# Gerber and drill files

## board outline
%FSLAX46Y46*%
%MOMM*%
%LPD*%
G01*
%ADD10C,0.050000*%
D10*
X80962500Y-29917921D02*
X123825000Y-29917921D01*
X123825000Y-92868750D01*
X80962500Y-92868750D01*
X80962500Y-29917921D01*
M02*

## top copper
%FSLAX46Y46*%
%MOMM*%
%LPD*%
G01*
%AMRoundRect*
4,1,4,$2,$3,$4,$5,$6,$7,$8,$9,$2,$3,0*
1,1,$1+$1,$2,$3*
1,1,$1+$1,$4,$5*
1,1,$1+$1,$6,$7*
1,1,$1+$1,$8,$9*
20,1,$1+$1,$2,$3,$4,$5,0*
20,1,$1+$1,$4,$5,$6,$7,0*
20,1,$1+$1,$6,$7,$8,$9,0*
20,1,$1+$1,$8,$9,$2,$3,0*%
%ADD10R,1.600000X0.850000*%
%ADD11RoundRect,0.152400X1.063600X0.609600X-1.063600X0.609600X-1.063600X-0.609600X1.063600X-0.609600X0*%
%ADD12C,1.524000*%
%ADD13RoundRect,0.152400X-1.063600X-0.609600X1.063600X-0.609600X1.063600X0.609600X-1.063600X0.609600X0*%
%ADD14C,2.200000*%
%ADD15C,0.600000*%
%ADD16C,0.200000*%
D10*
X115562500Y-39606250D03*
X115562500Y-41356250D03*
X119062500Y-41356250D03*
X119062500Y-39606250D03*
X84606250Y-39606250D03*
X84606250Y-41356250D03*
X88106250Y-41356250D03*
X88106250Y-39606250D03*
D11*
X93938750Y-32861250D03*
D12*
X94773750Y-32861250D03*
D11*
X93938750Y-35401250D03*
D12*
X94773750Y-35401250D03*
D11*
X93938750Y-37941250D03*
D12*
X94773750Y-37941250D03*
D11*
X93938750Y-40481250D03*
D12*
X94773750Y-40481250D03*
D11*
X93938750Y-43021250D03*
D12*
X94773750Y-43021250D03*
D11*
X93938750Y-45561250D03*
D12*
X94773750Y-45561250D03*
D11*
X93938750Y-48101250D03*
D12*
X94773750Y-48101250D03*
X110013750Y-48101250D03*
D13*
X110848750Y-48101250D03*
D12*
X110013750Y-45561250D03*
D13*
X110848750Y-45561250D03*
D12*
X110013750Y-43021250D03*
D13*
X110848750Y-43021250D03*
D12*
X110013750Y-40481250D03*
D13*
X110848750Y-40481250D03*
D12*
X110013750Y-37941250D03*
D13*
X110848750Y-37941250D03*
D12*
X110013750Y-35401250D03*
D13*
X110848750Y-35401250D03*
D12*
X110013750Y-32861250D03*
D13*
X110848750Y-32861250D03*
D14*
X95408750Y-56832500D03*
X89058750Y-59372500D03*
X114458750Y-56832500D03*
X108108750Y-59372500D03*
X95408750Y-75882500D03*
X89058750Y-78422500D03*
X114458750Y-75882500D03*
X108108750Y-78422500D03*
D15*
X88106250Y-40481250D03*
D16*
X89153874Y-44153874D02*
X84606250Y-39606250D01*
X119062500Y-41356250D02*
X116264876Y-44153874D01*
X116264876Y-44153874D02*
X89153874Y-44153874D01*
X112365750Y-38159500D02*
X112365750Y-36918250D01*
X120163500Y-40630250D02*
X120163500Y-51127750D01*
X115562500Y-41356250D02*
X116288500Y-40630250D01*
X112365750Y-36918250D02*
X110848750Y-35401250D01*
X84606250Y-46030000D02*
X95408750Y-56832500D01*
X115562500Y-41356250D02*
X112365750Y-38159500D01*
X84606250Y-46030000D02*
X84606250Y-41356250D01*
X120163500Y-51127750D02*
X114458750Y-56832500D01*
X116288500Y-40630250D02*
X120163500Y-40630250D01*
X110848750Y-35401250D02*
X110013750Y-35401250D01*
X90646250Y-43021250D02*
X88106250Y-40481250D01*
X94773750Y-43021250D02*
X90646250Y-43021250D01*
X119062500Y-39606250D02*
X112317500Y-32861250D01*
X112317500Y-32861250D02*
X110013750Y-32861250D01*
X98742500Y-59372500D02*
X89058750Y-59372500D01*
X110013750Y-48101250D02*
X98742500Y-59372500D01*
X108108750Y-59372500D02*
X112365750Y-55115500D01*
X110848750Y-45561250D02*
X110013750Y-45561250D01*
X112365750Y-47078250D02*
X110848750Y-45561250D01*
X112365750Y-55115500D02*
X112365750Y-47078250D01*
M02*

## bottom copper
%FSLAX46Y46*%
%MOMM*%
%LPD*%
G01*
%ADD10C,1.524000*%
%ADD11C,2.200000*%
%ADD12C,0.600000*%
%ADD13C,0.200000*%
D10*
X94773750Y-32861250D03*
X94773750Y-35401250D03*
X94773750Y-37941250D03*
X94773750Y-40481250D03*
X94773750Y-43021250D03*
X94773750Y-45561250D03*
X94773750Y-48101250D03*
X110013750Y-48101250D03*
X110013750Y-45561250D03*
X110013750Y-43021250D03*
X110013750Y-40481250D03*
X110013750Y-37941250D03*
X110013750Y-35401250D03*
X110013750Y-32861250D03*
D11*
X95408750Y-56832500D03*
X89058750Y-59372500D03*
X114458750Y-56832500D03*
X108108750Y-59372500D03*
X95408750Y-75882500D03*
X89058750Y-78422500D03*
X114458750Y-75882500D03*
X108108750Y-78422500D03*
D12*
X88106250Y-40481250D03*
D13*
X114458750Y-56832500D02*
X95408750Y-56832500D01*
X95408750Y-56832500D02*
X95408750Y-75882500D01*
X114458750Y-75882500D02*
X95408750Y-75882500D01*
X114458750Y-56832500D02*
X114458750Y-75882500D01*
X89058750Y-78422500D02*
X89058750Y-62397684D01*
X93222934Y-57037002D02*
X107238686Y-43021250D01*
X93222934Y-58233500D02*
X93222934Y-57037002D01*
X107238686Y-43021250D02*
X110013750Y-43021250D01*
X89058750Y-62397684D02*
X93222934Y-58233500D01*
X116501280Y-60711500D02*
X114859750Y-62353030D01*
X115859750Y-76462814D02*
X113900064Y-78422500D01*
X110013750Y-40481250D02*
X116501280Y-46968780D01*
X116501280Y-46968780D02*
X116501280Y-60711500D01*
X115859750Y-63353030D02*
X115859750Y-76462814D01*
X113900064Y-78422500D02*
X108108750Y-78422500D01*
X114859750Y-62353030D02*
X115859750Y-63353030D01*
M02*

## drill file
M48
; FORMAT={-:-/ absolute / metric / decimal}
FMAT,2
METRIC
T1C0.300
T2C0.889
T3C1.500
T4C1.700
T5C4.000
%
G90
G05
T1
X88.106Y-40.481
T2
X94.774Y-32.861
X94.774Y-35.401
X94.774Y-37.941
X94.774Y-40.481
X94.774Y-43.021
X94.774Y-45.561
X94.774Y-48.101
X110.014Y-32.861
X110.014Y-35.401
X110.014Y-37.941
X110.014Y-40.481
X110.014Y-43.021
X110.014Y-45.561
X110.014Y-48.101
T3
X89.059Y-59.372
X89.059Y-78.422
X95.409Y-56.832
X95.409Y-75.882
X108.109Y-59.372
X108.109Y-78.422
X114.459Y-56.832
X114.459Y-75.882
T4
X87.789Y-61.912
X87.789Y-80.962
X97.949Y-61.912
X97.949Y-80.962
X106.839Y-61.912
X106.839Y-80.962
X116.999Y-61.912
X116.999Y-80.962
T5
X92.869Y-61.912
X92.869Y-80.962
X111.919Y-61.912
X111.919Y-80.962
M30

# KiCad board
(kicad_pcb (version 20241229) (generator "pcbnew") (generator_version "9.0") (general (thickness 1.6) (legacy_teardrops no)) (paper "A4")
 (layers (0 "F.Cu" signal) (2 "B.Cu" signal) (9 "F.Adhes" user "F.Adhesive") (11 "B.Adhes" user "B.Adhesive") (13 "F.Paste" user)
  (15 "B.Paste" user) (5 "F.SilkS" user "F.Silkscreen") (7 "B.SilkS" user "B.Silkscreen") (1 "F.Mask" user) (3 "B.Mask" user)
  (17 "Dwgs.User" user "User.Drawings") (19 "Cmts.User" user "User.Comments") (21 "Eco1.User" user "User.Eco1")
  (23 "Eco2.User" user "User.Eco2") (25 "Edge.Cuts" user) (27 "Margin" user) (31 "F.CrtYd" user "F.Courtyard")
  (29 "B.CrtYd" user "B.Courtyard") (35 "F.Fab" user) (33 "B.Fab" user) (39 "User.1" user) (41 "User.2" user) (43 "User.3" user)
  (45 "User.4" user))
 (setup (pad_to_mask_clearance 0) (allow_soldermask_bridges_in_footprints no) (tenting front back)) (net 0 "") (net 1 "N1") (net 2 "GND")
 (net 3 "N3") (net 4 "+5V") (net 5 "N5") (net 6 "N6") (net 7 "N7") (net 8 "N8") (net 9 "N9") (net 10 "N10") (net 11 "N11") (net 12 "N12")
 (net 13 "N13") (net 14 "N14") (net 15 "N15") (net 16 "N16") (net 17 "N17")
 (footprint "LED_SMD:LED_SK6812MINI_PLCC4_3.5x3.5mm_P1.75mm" (layer "F.Cu") (at 117.3125 40.48125)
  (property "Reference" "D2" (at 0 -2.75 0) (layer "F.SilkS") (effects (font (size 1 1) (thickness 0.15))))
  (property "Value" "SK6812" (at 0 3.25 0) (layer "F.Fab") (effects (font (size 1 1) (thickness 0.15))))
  (pad "1" smd rect (at -1.75 -0.875) (size 1.6 0.85) (layers "F.Cu" "F.Mask" "F.Paste") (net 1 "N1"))
  (pad "2" smd rect (at -1.75 0.875) (size 1.6 0.85) (layers "F.Cu" "F.Mask" "F.Paste") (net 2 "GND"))
  (pad "3" smd rect (at 1.75 0.875) (size 1.6 0.85) (layers "F.Cu" "F.Mask" "F.Paste") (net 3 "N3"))
  (pad "4" smd rect (at 1.75 -0.875) (size 1.6 0.85) (layers "F.Cu" "F.Mask" "F.Paste") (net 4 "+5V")))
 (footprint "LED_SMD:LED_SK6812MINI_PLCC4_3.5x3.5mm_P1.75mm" (layer "F.Cu") (at 86.35625 40.48125)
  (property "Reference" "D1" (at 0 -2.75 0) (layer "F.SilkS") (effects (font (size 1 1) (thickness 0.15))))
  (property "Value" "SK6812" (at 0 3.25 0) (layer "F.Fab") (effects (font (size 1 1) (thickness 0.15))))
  (pad "1" smd rect (at -1.75 -0.875) (size 1.6 0.85) (layers "F.Cu" "F.Mask" "F.Paste") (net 3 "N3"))
  (pad "2" smd rect (at -1.75 0.875) (size 1.6 0.85) (layers "F.Cu" "F.Mask" "F.Paste") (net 2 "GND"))
  (pad "3" smd rect (at 1.75 0.875) (size 1.6 0.85) (layers "F.Cu" "F.Mask" "F.Paste") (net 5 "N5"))
  (pad "4" smd rect (at 1.75 -0.875) (size 1.6 0.85) (layers "F.Cu" "F.Mask" "F.Paste") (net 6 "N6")))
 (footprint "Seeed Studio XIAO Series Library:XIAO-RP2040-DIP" (layer "F.Cu") (at 102.39375 40.48125)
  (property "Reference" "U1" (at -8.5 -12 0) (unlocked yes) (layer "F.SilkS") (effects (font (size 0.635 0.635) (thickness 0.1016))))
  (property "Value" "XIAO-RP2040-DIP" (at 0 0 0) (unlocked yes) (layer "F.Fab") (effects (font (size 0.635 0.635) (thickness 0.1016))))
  (pad "1" smd roundrect (at -8.455 -7.62 180) (size 2.432 1.524) (layers "F.Cu" "F.Mask") (roundrect_rratio 0.1) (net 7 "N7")
   (thermal_bridge_angle 45))
  (pad "1" thru_hole circle (at -7.62 -7.62 180) (size 1.524 1.524) (drill 0.889) (layers "*.Cu" "*.Mask") (remove_unused_layers no)
   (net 7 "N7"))
  (pad "2" smd roundrect (at -8.455 -5.08 180) (size 2.432 1.524) (layers "F.Cu" "F.Mask") (roundrect_rratio 0.1) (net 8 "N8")
   (thermal_bridge_angle 45))
  (pad "2" thru_hole circle (at -7.62 -5.08 180) (size 1.524 1.524) (drill 0.889) (layers "*.Cu" "*.Mask") (remove_unused_layers no)
   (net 8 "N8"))
  (pad "3" smd roundrect (at -8.455 -2.54 180) (size 2.432 1.524) (layers "F.Cu" "F.Mask") (roundrect_rratio 0.1) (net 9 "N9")
   (thermal_bridge_angle 45))
  (pad "3" thru_hole circle (at -7.62 -2.54 180) (size 1.524 1.524) (drill 0.889) (layers "*.Cu" "*.Mask") (remove_unused_layers no)
   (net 9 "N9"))
  (pad "4" smd roundrect (at -8.455 0 180) (size 2.432 1.524) (layers "F.Cu" "F.Mask") (roundrect_rratio 0.1) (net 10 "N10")
   (thermal_bridge_angle 45))
  (pad "4" thru_hole circle (at -7.62 0 180) (size 1.524 1.524) (drill 0.889) (layers "*.Cu" "*.Mask") (remove_unused_layers no)
   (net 10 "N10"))
  (pad "5" smd roundrect (at -8.455 2.54 180) (size 2.432 1.524) (layers "F.Cu" "F.Mask") (roundrect_rratio 0.1) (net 5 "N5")
   (thermal_bridge_angle 45))
  (pad "5" thru_hole circle (at -7.62 2.54 180) (size 1.524 1.524) (drill 0.889) (layers "*.Cu" "*.Mask") (remove_unused_layers no)
   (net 5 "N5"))
  (pad "6" smd roundrect (at -8.455 5.08 180) (size 2.432 1.524) (layers "F.Cu" "F.Mask") (roundrect_rratio 0.1) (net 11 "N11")
   (thermal_bridge_angle 45))
  (pad "6" thru_hole circle (at -7.62 5.08 180) (size 1.524 1.524) (drill 0.889) (layers "*.Cu" "*.Mask") (remove_unused_layers no)
   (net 11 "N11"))
  (pad "7" smd roundrect (at -8.455 7.62 180) (size 2.432 1.524) (layers "F.Cu" "F.Mask") (roundrect_rratio 0.1) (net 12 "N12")
   (thermal_bridge_angle 45))
  (pad "7" thru_hole circle (at -7.62 7.62 180) (size 1.524 1.524) (drill 0.889) (layers "*.Cu" "*.Mask") (remove_unused_layers no)
   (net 12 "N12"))
  (pad "8" thru_hole circle (at 7.62 7.62) (size 1.524 1.524) (drill 0.889) (layers "*.Cu" "*.Mask") (remove_unused_layers no)
   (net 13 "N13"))
  (pad "8" smd roundrect (at 8.455 7.62) (size 2.432 1.524) (layers "F.Cu" "F.Mask") (roundrect_rratio 0.1) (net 13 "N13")
   (thermal_bridge_angle 45))
  (pad "9" thru_hole circle (at 7.62 5.08) (size 1.524 1.524) (drill 0.889) (layers "*.Cu" "*.Mask") (remove_unused_layers no)
   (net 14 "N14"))
  (pad "9" smd roundrect (at 8.455 5.08) (size 2.432 1.524) (layers "F.Cu" "F.Mask") (roundrect_rratio 0.1) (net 14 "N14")
   (thermal_bridge_angle 45))
  (pad "10" thru_hole circle (at 7.62 2.54) (size 1.524 1.524) (drill 0.889) (layers "*.Cu" "*.Mask") (remove_unused_layers no)
   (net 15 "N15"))
  (pad "10" smd roundrect (at 8.455 2.54) (size 2.432 1.524) (layers "F.Cu" "F.Mask") (roundrect_rratio 0.1) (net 15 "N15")
   (thermal_bridge_angle 45))
  (pad "11" thru_hole circle (at 7.62 0) (size 1.524 1.524) (drill 0.889) (layers "*.Cu" "*.Mask") (remove_unused_layers no) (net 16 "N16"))
  (pad "11" smd roundrect (at 8.455 0) (size 2.432 1.524) (layers "F.Cu" "F.Mask") (roundrect_rratio 0.1) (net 16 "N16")
   (thermal_bridge_angle 45))
  (pad "12" thru_hole circle (at 7.62 -2.54) (size 1.524 1.524) (drill 0.889) (layers "*.Cu" "*.Mask") (remove_unused_layers no)
   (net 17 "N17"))
  (pad "12" smd roundrect (at 8.455 -2.54) (size 2.432 1.524) (layers "F.Cu" "F.Mask") (roundrect_rratio 0.1) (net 17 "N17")
   (thermal_bridge_angle 45))
  (pad "13" thru_hole circle (at 7.62 -5.08) (size 1.524 1.524) (drill 0.889) (layers "*.Cu" "*.Mask") (remove_unused_layers no)
   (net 2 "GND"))
  (pad "13" smd roundrect (at 8.455 -5.08) (size 2.432 1.524) (layers "F.Cu" "F.Mask") (roundrect_rratio 0.1) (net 2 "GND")
   (thermal_bridge_angle 45))
  (pad "14" thru_hole circle (at 7.62 -7.62) (size 1.524 1.524) (drill 0.889) (layers "*.Cu" "*.Mask") (remove_unused_layers no)
   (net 4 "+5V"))
  (pad "14" smd roundrect (at 8.455 -7.62) (size 2.432 1.524) (layers "F.Cu" "F.Mask") (roundrect_rratio 0.1) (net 4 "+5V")
   (thermal_bridge_angle 45)))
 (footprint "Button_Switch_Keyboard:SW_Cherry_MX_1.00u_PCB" (layer "F.Cu") (at 95.40875 56.8325)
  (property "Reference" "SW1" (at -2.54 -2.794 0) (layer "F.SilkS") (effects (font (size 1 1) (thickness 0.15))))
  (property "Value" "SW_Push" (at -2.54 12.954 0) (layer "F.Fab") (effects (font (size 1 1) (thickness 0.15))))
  (pad "" np_thru_hole circle (at -7.62 5.08) (size 1.7 1.7) (drill 1.7) (layers "*.Cu" "*.Mask"))
  (pad "" np_thru_hole circle (at -2.54 5.08) (size 4 4) (drill 4) (layers "*.Cu" "*.Mask"))
  (pad "" np_thru_hole circle (at 2.54 5.08) (size 1.7 1.7) (drill 1.7) (layers "*.Cu" "*.Mask"))
  (pad "1" thru_hole circle (at 0 0) (size 2.2 2.2) (drill 1.5) (layers "*.Cu" "*.Mask") (remove_unused_layers no) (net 2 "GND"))
  (pad "2" thru_hole circle (at -6.35 2.54) (size 2.2 2.2) (drill 1.5) (layers "*.Cu" "*.Mask") (remove_unused_layers no) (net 13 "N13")))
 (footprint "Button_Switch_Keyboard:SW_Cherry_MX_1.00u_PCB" (layer "F.Cu") (at 114.45875 56.8325)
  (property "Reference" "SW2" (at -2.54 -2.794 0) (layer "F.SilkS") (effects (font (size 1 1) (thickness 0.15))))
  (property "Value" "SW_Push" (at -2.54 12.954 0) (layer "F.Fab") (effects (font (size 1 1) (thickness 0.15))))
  (pad "" np_thru_hole circle (at -7.62 5.08) (size 1.7 1.7) (drill 1.7) (layers "*.Cu" "*.Mask"))
  (pad "" np_thru_hole circle (at -2.54 5.08) (size 4 4) (drill 4) (layers "*.Cu" "*.Mask"))
  (pad "" np_thru_hole circle (at 2.54 5.08) (size 1.7 1.7) (drill 1.7) (layers "*.Cu" "*.Mask"))
  (pad "1" thru_hole circle (at 0 0) (size 2.2 2.2) (drill 1.5) (layers "*.Cu" "*.Mask") (remove_unused_layers no) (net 2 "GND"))
  (pad "2" thru_hole circle (at -6.35 2.54) (size 2.2 2.2) (drill 1.5) (layers "*.Cu" "*.Mask") (remove_unused_layers no) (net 14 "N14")))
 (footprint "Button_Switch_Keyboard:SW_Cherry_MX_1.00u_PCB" (layer "F.Cu") (at 95.40875 75.8825)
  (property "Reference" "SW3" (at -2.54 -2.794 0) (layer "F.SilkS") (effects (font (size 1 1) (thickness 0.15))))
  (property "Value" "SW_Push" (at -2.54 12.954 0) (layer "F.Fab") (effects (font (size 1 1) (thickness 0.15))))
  (pad "" np_thru_hole circle (at -7.62 5.08) (size 1.7 1.7) (drill 1.7) (layers "*.Cu" "*.Mask"))
  (pad "" np_thru_hole circle (at -2.54 5.08) (size 4 4) (drill 4) (layers "*.Cu" "*.Mask"))
  (pad "" np_thru_hole circle (at 2.54 5.08) (size 1.7 1.7) (drill 1.7) (layers "*.Cu" "*.Mask"))
  (pad "1" thru_hole circle (at 0 0) (size 2.2 2.2) (drill 1.5) (layers "*.Cu" "*.Mask") (remove_unused_layers no) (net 2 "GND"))
  (pad "2" thru_hole circle (at -6.35 2.54) (size 2.2 2.2) (drill 1.5) (layers "*.Cu" "*.Mask") (remove_unused_layers no) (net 15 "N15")))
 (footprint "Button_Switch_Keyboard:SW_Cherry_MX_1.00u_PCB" (layer "F.Cu") (at 114.45875 75.8825)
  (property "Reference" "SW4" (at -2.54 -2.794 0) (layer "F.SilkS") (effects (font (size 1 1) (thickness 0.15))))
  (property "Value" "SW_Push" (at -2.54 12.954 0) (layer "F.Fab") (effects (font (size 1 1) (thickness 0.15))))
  (pad "" np_thru_hole circle (at -7.62 5.08) (size 1.7 1.7) (drill 1.7) (layers "*.Cu" "*.Mask"))
  (pad "" np_thru_hole circle (at -2.54 5.08) (size 4 4) (drill 4) (layers "*.Cu" "*.Mask"))
  (pad "" np_thru_hole circle (at 2.54 5.08) (size 1.7 1.7) (drill 1.7) (layers "*.Cu" "*.Mask"))
  (pad "1" thru_hole circle (at 0 0) (size 2.2 2.2) (drill 1.5) (layers "*.Cu" "*.Mask") (remove_unused_layers no) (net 2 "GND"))
  (pad "2" thru_hole circle (at -6.35 2.54) (size 2.2 2.2) (drill 1.5) (layers "*.Cu" "*.Mask") (remove_unused_layers no) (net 16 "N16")))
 (gr_rect (start 80.9625 29.917921) (end 123.825 92.86875) (stroke (width 0.05) (type default)) (fill no) (layer "Edge.Cuts"))
 (segment (start 89.153874 44.153874) (end 84.60625 39.60625) (width 0.2) (layer "F.Cu") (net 3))
 (segment (start 119.0625 41.35625) (end 116.264876 44.153874) (width 0.2) (layer "F.Cu") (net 3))
 (segment (start 116.264876 44.153874) (end 89.153874 44.153874) (width 0.2) (layer "F.Cu") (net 3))
 (segment (start 112.36575 38.1595) (end 112.36575 36.91825) (width 0.2) (layer "F.Cu") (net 2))
 (segment (start 120.1635 40.63025) (end 120.1635 51.12775) (width 0.2) (layer "F.Cu") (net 2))
 (segment (start 115.5625 41.35625) (end 116.2885 40.63025) (width 0.2) (layer "F.Cu") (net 2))
 (segment (start 112.36575 36.91825) (end 110.84875 35.40125) (width 0.2) (layer "F.Cu") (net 2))
 (segment (start 84.60625 46.03) (end 95.40875 56.8325) (width 0.2) (layer "F.Cu") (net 2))
 (segment (start 115.5625 41.35625) (end 112.36575 38.1595) (width 0.2) (layer "F.Cu") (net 2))
 (segment (start 84.60625 46.03) (end 84.60625 41.35625) (width 0.2) (layer "F.Cu") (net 2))
 (segment (start 120.1635 51.12775) (end 114.45875 56.8325) (width 0.2) (layer "F.Cu") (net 2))
 (segment (start 116.2885 40.63025) (end 120.1635 40.63025) (width 0.2) (layer "F.Cu") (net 2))
 (segment (start 110.84875 35.40125) (end 110.01375 35.40125) (width 0.2) (layer "F.Cu") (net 2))
 (segment (start 114.45875 56.8325) (end 95.40875 56.8325) (width 0.2) (layer "B.Cu") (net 2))
 (segment (start 95.40875 56.8325) (end 95.40875 75.8825) (width 0.2) (layer "B.Cu") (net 2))
 (segment (start 114.45875 75.8825) (end 95.40875 75.8825) (width 0.2) (layer "B.Cu") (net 2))
 (segment (start 114.45875 56.8325) (end 114.45875 75.8825) (width 0.2) (layer "B.Cu") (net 2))
 (segment (start 90.64625 43.02125) (end 88.10625 40.48125) (width 0.2) (layer "F.Cu") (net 5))
 (segment (start 94.77375 43.02125) (end 90.64625 43.02125) (width 0.2) (layer "F.Cu") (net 5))
 (via (at 88.10625 40.48125) (size 0.6) (drill 0.3) (layers "F.Cu" "B.Cu") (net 5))
 (segment (start 119.0625 39.60625) (end 112.3175 32.86125) (width 0.2) (layer "F.Cu") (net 4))
 (segment (start 112.3175 32.86125) (end 110.01375 32.86125) (width 0.2) (layer "F.Cu") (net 4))
 (segment (start 98.7425 59.3725) (end 89.05875 59.3725) (width 0.2) (layer "F.Cu") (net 13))
 (segment (start 110.01375 48.10125) (end 98.7425 59.3725) (width 0.2) (layer "F.Cu") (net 13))
 (segment (start 108.10875 59.3725) (end 112.36575 55.1155) (width 0.2) (layer "F.Cu") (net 14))
 (segment (start 110.84875 45.56125) (end 110.01375 45.56125) (width 0.2) (layer "F.Cu") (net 14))
 (segment (start 112.36575 47.07825) (end 110.84875 45.56125) (width 0.2) (layer "F.Cu") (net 14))
 (segment (start 112.36575 55.1155) (end 112.36575 47.07825) (width 0.2) (layer "F.Cu") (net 14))
 (segment (start 89.05875 78.4225) (end 89.05875 62.397684) (width 0.2) (layer "B.Cu") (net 15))
 (segment (start 93.222934 57.037002) (end 107.238686 43.02125) (width 0.2) (layer "B.Cu") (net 15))
 (segment (start 93.222934 58.2335) (end 93.222934 57.037002) (width 0.2) (layer "B.Cu") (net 15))
 (segment (start 107.238686 43.02125) (end 110.01375 43.02125) (width 0.2) (layer "B.Cu") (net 15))
 (segment (start 89.05875 62.397684) (end 93.222934 58.2335) (width 0.2) (layer "B.Cu") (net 15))
 (segment (start 116.50128 60.7115) (end 114.85975 62.35303) (width 0.2) (layer "B.Cu") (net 16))
 (segment (start 115.85975 76.462814) (end 113.900064 78.4225) (width 0.2) (layer "B.Cu") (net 16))
 (segment (start 110.01375 40.48125) (end 116.50128 46.96878) (width 0.2) (layer "B.Cu") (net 16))
 (segment (start 116.50128 46.96878) (end 116.50128 60.7115) (width 0.2) (layer "B.Cu") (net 16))
 (segment (start 115.85975 63.35303) (end 115.85975 76.462814) (width 0.2) (layer "B.Cu") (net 16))
 (segment (start 113.900064 78.4225) (end 108.10875 78.4225) (width 0.2) (layer "B.Cu") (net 16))
 (segment (start 114.85975 62.35303) (end 115.85975 63.35303) (width 0.2) (layer "B.Cu") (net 16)))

